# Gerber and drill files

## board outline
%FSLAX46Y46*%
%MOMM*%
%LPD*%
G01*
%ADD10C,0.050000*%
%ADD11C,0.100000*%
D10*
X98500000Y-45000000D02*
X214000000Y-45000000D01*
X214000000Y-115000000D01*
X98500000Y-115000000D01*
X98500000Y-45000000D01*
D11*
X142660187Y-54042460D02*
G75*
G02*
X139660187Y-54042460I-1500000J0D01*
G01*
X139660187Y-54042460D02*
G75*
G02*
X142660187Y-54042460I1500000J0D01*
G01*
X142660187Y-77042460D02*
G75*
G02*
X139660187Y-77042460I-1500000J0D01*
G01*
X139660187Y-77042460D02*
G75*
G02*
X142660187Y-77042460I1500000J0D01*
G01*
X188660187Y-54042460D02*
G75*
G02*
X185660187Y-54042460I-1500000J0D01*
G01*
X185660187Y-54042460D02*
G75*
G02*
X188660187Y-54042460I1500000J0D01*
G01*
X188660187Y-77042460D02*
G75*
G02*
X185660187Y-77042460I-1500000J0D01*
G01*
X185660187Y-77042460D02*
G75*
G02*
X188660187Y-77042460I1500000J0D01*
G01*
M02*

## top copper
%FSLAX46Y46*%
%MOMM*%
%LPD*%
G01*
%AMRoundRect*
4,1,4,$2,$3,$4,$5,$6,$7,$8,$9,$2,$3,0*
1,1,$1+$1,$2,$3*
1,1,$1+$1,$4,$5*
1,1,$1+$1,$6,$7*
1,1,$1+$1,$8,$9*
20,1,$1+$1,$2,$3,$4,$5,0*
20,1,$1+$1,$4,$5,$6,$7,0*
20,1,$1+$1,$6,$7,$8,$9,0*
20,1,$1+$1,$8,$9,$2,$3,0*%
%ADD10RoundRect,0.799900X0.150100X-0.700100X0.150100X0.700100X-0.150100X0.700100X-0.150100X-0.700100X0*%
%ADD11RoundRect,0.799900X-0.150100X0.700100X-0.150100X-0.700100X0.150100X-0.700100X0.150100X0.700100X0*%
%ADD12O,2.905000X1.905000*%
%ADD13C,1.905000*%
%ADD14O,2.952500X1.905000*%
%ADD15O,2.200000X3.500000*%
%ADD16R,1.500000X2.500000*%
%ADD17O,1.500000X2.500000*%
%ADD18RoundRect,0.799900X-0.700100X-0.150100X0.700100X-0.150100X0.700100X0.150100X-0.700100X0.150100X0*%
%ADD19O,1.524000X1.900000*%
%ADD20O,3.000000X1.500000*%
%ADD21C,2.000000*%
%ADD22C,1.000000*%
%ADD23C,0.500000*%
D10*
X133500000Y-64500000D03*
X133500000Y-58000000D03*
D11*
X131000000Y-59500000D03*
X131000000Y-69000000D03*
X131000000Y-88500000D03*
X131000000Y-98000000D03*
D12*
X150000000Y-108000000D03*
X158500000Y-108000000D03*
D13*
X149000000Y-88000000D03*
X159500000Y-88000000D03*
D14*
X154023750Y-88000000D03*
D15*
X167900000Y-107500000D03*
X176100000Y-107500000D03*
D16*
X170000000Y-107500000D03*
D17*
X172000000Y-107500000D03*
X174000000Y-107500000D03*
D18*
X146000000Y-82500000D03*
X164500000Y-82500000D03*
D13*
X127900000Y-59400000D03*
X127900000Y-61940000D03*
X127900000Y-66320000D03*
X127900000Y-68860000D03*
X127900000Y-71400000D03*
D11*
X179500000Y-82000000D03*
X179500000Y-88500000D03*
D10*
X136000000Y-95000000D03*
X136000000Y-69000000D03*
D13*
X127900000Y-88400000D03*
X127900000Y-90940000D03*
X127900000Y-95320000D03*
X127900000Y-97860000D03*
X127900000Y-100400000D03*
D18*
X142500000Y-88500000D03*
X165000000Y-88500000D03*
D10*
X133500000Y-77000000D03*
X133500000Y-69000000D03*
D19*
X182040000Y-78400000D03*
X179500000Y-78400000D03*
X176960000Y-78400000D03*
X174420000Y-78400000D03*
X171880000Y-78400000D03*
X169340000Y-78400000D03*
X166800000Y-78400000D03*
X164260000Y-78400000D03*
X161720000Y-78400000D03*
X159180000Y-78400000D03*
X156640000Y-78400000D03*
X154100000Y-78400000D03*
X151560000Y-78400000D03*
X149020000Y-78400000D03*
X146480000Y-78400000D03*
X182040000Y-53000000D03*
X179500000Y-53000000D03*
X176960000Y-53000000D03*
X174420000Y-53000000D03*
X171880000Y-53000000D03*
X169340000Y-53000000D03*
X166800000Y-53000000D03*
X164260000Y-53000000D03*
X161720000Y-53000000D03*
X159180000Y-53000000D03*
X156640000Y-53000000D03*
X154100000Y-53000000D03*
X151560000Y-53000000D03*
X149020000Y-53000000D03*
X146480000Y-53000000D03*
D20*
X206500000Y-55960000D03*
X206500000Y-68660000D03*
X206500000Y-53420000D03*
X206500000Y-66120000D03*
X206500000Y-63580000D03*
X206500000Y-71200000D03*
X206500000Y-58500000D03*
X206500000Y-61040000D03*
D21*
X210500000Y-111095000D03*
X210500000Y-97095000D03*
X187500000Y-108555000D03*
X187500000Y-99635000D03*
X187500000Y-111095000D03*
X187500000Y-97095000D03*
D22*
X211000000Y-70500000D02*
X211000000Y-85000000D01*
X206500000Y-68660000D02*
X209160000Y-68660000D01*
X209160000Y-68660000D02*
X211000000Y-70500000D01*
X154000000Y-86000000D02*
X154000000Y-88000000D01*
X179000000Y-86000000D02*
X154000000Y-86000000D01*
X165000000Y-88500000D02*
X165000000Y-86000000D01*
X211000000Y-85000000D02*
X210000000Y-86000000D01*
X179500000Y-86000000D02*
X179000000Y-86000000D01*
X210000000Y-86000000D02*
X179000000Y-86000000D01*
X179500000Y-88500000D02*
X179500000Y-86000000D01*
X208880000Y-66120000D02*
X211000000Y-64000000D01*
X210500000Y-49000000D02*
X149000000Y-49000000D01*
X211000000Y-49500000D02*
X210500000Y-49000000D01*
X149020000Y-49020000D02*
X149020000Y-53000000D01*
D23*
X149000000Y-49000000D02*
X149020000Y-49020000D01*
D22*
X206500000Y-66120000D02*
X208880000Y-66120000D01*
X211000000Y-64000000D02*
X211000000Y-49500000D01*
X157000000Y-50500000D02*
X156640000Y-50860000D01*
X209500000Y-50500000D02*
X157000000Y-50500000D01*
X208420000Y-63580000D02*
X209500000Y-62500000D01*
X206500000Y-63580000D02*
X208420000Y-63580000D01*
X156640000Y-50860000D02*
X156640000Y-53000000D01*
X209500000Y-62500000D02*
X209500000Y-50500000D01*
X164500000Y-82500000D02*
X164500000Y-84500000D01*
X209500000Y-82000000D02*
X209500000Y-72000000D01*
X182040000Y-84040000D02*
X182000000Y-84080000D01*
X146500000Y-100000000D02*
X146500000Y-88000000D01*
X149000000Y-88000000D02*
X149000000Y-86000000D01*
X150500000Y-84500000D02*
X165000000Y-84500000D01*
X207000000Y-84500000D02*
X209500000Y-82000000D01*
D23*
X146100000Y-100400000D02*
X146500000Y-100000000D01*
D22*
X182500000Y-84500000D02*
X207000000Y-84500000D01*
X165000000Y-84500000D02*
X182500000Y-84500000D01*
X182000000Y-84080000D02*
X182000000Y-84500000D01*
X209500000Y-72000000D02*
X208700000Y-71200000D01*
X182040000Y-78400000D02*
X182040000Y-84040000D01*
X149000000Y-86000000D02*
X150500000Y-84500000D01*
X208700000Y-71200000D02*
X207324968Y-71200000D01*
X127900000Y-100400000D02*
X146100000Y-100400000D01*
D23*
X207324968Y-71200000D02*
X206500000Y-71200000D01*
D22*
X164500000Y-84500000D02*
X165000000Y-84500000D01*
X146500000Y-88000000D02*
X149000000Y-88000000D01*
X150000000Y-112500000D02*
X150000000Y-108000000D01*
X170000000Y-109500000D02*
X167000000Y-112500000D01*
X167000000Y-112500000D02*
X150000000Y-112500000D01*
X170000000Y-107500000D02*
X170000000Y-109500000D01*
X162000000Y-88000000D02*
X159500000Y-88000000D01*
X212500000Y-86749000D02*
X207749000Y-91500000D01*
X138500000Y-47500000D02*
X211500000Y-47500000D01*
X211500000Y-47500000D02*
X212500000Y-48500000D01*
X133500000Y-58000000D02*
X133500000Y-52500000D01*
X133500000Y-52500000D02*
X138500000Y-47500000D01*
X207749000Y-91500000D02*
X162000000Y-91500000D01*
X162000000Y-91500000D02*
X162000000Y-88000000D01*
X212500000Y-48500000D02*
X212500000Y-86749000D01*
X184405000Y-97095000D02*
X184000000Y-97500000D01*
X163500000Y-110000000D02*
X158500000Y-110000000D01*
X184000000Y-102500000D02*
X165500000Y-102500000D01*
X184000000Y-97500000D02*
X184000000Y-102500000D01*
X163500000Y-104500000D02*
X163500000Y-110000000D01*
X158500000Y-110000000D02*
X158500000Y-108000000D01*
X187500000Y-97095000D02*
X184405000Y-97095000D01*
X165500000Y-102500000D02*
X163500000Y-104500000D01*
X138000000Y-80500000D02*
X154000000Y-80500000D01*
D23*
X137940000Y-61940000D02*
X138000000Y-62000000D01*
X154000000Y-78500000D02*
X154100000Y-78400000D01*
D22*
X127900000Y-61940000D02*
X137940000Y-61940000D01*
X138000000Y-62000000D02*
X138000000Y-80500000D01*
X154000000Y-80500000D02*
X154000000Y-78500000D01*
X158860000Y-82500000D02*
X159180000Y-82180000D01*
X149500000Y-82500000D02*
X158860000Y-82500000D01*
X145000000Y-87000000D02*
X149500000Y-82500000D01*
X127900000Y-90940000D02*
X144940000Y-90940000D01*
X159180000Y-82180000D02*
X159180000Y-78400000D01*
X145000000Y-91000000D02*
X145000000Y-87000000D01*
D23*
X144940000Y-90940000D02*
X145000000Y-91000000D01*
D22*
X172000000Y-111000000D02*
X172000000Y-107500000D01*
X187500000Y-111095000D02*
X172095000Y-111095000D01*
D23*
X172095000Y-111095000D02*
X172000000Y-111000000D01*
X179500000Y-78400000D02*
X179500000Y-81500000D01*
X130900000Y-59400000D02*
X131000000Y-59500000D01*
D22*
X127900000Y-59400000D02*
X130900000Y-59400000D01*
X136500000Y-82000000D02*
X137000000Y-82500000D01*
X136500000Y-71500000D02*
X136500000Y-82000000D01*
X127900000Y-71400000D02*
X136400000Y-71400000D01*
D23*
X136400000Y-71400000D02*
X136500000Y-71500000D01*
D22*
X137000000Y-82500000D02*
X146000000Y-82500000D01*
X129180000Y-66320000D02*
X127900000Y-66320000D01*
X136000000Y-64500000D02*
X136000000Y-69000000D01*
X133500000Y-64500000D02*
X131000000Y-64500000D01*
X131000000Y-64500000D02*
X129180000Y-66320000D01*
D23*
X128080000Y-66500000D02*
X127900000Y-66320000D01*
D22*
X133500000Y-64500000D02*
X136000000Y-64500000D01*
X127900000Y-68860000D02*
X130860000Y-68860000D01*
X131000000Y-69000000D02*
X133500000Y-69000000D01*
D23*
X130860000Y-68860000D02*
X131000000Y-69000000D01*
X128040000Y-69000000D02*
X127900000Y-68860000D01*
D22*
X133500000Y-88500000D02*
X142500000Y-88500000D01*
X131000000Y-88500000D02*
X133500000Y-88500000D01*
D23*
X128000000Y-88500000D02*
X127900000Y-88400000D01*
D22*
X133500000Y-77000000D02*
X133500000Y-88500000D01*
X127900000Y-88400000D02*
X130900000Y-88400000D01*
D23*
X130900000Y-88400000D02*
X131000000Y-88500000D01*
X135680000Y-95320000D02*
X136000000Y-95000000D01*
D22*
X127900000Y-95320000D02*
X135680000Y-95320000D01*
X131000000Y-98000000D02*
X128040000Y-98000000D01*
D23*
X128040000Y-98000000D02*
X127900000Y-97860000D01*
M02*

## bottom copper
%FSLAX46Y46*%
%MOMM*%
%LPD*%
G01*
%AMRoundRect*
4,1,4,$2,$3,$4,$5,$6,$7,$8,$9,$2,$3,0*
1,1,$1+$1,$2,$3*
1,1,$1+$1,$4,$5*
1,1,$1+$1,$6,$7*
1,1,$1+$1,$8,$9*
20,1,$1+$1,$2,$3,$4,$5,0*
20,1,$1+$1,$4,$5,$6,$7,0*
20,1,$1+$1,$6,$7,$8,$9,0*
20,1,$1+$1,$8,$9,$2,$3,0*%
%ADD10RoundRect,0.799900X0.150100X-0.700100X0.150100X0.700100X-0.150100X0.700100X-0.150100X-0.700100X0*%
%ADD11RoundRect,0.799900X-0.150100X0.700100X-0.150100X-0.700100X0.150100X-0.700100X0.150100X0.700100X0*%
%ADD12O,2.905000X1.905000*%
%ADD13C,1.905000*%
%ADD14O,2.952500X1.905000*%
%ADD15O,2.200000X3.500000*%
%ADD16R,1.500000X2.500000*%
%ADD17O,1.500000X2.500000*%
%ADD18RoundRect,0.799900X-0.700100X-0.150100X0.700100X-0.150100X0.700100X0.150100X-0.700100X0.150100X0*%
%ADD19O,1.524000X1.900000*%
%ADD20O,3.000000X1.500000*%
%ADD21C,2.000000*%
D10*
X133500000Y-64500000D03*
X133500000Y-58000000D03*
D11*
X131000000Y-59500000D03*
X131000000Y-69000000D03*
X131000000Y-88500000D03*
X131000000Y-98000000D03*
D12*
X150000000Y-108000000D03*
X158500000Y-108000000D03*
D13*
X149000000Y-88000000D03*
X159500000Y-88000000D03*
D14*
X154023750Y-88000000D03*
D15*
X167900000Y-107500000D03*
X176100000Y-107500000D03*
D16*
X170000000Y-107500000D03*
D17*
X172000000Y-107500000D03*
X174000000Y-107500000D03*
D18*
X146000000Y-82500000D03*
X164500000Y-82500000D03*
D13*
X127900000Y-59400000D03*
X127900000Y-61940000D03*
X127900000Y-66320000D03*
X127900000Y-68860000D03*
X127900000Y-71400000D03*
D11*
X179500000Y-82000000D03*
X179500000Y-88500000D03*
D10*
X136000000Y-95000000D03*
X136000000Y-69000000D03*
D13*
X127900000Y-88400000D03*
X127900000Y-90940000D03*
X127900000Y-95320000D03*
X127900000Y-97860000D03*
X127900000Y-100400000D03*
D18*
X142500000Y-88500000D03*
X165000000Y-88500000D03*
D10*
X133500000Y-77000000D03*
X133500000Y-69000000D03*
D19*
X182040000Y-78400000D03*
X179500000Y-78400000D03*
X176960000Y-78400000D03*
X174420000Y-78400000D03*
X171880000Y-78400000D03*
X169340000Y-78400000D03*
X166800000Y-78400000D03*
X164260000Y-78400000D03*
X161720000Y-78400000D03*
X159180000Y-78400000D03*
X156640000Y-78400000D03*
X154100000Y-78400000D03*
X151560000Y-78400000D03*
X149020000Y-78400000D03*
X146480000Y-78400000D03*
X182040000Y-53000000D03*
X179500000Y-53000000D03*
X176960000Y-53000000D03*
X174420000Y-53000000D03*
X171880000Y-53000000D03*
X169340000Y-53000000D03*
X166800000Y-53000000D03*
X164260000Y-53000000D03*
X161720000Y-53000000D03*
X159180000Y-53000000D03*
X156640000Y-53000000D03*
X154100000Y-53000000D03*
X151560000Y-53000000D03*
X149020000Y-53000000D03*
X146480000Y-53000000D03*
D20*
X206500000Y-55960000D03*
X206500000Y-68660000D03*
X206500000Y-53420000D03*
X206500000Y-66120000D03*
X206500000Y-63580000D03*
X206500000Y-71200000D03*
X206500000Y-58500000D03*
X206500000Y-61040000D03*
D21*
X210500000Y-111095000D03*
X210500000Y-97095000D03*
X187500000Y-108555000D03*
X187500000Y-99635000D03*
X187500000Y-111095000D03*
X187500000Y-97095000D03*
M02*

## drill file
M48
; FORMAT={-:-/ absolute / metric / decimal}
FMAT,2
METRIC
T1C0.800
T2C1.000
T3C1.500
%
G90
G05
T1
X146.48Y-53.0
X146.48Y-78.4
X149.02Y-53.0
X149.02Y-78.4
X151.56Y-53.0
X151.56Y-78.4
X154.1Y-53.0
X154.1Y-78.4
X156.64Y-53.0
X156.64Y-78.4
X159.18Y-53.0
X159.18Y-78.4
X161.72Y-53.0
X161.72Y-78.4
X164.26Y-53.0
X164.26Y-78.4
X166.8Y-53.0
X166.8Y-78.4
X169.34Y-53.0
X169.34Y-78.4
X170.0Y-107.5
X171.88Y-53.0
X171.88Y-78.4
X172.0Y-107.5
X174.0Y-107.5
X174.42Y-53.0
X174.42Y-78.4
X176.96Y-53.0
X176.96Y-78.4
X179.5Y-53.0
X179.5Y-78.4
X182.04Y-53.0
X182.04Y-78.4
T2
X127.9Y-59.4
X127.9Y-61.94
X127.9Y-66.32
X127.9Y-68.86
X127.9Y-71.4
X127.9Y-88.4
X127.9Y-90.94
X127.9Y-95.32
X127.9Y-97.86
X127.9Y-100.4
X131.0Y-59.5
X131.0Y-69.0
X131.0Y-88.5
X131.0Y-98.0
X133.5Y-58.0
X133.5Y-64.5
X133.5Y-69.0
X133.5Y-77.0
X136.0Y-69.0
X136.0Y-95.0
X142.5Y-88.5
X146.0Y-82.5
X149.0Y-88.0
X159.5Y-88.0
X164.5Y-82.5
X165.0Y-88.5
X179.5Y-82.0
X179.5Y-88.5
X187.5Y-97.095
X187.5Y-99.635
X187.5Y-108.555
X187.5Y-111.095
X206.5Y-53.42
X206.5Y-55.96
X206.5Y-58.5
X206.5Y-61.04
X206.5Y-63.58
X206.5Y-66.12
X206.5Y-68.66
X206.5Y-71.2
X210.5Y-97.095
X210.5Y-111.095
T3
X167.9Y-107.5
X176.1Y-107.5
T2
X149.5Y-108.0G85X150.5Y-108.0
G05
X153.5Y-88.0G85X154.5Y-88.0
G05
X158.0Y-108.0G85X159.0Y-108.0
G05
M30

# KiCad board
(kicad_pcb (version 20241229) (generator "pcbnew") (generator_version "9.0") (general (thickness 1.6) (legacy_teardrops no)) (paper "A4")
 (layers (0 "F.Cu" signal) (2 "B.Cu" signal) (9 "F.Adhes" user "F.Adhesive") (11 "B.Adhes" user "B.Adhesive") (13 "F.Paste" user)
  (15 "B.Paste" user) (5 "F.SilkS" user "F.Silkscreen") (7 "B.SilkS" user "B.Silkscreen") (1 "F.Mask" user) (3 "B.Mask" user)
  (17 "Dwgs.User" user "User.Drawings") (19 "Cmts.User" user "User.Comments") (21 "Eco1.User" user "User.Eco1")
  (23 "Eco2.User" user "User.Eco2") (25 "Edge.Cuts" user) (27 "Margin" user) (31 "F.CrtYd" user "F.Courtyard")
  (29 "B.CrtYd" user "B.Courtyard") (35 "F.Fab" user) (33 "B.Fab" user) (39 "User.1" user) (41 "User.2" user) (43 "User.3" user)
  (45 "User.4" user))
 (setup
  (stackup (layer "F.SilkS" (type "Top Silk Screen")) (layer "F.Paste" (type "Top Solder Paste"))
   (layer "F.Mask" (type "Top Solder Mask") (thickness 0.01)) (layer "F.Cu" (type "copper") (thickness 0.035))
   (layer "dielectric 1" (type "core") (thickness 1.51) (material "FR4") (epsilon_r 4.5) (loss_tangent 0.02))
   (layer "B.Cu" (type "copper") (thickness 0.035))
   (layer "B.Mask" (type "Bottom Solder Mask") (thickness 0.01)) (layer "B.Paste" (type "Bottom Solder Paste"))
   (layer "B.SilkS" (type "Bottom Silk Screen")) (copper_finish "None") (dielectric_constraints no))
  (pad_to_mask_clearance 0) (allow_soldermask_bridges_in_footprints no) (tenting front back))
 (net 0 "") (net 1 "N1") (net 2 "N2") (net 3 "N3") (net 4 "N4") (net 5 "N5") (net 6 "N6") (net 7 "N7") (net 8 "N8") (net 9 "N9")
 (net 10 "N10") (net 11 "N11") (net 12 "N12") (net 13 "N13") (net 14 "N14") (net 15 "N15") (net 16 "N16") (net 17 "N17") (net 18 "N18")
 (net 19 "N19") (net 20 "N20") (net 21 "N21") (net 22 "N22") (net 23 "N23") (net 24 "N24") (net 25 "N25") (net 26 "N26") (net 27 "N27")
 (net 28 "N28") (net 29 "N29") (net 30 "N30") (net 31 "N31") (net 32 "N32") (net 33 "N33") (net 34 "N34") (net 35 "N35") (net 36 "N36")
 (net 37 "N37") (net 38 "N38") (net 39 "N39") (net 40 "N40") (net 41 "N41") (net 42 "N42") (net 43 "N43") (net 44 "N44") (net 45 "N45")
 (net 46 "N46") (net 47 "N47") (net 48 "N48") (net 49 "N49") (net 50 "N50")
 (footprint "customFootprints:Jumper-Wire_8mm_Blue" (layer "F.Cu") (at 133.5 66 90)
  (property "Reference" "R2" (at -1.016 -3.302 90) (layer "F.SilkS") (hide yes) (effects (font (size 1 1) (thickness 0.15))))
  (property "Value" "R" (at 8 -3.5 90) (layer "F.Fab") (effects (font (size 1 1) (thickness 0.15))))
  (pad "1" thru_hole roundrect (at 1.5 0 90) (size 3 1.9) (drill 1) (layers "*.Cu") (remove_unused_layers no) (roundrect_rratio 0.421)
   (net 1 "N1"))
  (pad "2" thru_hole roundrect (at 8 0 90) (size 3 1.9) (drill 1) (layers "*.Cu") (remove_unused_layers no) (roundrect_rratio 0.421)
   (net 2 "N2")))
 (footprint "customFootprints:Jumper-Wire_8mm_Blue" (layer "F.Cu") (at 131 59.5 -90)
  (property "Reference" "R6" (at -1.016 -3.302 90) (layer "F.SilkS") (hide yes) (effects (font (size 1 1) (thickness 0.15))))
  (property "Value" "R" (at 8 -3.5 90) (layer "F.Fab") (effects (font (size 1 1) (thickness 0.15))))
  (pad "1" thru_hole roundrect (at 0 0 270) (size 3 1.9) (drill 1) (layers "*.Cu") (remove_unused_layers no) (roundrect_rratio 0.421)
   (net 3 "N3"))
  (pad "2" thru_hole roundrect (at 9.5 0 270) (size 3 1.9) (drill 1) (layers "*.Cu") (remove_unused_layers no) (roundrect_rratio 0.421)
   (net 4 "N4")))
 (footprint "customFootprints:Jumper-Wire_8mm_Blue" (layer "F.Cu") (at 131 88.5 -90)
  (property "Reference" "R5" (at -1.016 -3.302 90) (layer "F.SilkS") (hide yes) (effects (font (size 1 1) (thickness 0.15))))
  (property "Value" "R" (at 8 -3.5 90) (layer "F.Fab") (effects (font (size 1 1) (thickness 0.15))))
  (pad "1" thru_hole roundrect (at 0 0 270) (size 3 1.9) (drill 1) (layers "*.Cu") (remove_unused_layers no) (roundrect_rratio 0.421)
   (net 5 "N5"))
  (pad "2" thru_hole roundrect (at 9.5 0 270) (size 3 1.9) (drill 1) (layers "*.Cu") (remove_unused_layers no) (roundrect_rratio 0.421)
   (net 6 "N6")))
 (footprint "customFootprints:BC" (layer "F.Cu") (at 154.5 98 90)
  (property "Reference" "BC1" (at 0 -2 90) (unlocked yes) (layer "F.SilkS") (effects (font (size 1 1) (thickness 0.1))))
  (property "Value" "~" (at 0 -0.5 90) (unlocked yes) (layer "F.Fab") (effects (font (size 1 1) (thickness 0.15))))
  (pad "1" thru_hole oval (at -10 -4.5 90) (size 1.905 2.905) (drill oval 1 2) (layers "*.Cu" "*.Mask") (remove_unused_layers no)
   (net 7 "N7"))
  (pad "2" thru_hole oval (at -10 4 90) (size 1.905 2.905) (drill oval 1 2) (layers "*.Cu" "*.Mask") (remove_unused_layers no) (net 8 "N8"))
  (pad "3" thru_hole circle (at 10 -5.5 90) (size 1.905 1.905) (drill 1) (layers "*.Cu" "*.Mask") (remove_unused_layers no) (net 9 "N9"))
  (pad "4" thru_hole circle (at 10 5 90) (size 1.905 1.905) (drill 1) (layers "*.Cu" "*.Mask") (remove_unused_layers no) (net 2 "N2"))
  (pad "5" thru_hole oval (at 10 -0.5 90) (size 1.905 2.9525) (drill oval 1 2 (offset 0 0.02375)) (layers "*.Cu" "*.Mask")
   (remove_unused_layers no) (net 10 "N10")))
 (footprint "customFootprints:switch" (layer "F.Cu") (at 170 107.5)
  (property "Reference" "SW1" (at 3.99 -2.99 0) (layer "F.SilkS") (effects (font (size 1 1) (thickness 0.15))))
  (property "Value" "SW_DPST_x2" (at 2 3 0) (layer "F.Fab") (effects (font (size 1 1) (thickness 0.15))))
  (pad "" thru_hole oval (at -2.1 0) (size 2.2 3.5) (drill 1.5) (layers "*.Cu" "*.Mask") (remove_unused_layers no))
  (pad "" thru_hole oval (at 6.1 0) (size 2.2 3.5) (drill 1.5) (layers "*.Cu" "*.Mask") (remove_unused_layers no))
  (pad "1" thru_hole rect (at 0 0) (size 1.5 2.5) (drill 0.8) (layers "*.Cu" "*.Mask") (remove_unused_layers no) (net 7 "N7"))
  (pad "2" thru_hole oval (at 2 0) (size 1.5 2.5) (drill 0.8) (layers "*.Cu" "*.Mask") (remove_unused_layers no) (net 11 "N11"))
  (pad "3" thru_hole oval (at 4 0) (size 1.5 2.5) (drill 0.8) (layers "*.Cu" "*.Mask") (remove_unused_layers no)))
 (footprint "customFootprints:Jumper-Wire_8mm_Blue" (layer "F.Cu") (at 146 82.5)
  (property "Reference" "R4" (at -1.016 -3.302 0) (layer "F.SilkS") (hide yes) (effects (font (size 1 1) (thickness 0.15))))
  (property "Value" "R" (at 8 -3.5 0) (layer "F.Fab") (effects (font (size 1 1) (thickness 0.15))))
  (pad "1" thru_hole roundrect (at 0 0) (size 3 1.9) (drill 1) (layers "*.Cu") (remove_unused_layers no) (roundrect_rratio 0.421)
   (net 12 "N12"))
  (pad "2" thru_hole roundrect (at 18.5 0) (size 3 1.9) (drill 1) (layers "*.Cu") (remove_unused_layers no) (roundrect_rratio 0.421)
   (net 9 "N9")))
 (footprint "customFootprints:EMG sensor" (layer "F.Cu") (at 129.4 79.4 180)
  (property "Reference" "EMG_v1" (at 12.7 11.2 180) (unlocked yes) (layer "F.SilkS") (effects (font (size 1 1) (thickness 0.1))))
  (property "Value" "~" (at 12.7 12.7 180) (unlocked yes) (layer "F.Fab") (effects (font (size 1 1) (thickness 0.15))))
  (pad "1" thru_hole circle (at 1.5 20 180) (size 1.905 1.905) (drill 1) (layers "*.Cu" "*.Mask") (remove_unused_layers no) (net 3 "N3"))
  (pad "2" thru_hole circle (at 1.5 17.46 180) (size 1.905 1.905) (drill 1) (layers "*.Cu" "*.Mask") (remove_unused_layers no)
   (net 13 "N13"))
  (pad "3" thru_hole circle (at 1.5 13.08 180) (size 1.905 1.905) (drill 1) (layers "*.Cu" "*.Mask") (remove_unused_layers no) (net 1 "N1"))
  (pad "4" thru_hole circle (at 1.5 10.54 180) (size 1.905 1.905) (drill 1) (layers "*.Cu" "*.Mask") (remove_unused_layers no) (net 4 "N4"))
  (pad "5" thru_hole circle (at 1.5 8 180) (size 1.905 1.905) (drill 1) (layers "*.Cu" "*.Mask") (remove_unused_layers no) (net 12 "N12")))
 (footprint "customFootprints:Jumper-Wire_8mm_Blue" (layer "F.Cu") (at 179.5 80.5 -90)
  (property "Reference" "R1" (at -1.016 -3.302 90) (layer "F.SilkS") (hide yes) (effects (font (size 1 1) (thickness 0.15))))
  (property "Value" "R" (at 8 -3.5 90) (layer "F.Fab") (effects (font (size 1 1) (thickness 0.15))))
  (pad "1" thru_hole roundrect (at 1.5 0 270) (size 3 1.9) (drill 1) (layers "*.Cu") (remove_unused_layers no) (roundrect_rratio 0.421)
   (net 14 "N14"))
  (pad "2" thru_hole roundrect (at 8 0 270) (size 3 1.9) (drill 1) (layers "*.Cu") (remove_unused_layers no) (roundrect_rratio 0.421)
   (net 10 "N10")))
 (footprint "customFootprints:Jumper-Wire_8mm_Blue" (layer "F.Cu") (at 136 95 90)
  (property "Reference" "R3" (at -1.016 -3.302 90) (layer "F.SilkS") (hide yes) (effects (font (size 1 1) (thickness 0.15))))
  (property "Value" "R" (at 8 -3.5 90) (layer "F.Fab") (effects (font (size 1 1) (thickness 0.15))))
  (pad "1" thru_hole roundrect (at 0 0 90) (size 3 1.9) (drill 1) (layers "*.Cu") (remove_unused_layers no) (roundrect_rratio 0.421)
   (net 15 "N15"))
  (pad "2" thru_hole roundrect (at 26 0 90) (size 3 1.9) (drill 1) (layers "*.Cu") (remove_unused_layers no) (roundrect_rratio 0.421)
   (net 1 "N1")))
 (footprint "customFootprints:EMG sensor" (layer "F.Cu") (at 129.4 108.4 180)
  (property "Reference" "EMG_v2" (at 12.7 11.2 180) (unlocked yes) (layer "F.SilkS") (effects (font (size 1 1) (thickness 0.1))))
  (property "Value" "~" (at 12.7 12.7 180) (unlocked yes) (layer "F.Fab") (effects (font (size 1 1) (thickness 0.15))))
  (pad "1" thru_hole circle (at 1.5 20 180) (size 1.905 1.905) (drill 1) (layers "*.Cu" "*.Mask") (remove_unused_layers no) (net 5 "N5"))
  (pad "2" thru_hole circle (at 1.5 17.46 180) (size 1.905 1.905) (drill 1) (layers "*.Cu" "*.Mask") (remove_unused_layers no)
   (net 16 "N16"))
  (pad "3" thru_hole circle (at 1.5 13.08 180) (size 1.905 1.905) (drill 1) (layers "*.Cu" "*.Mask") (remove_unused_layers no)
   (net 15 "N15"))
  (pad "4" thru_hole circle (at 1.5 10.54 180) (size 1.905 1.905) (drill 1) (layers "*.Cu" "*.Mask") (remove_unused_layers no) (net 6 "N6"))
  (pad "5" thru_hole circle (at 1.5 8 180) (size 1.905 1.905) (drill 1) (layers "*.Cu" "*.Mask") (remove_unused_layers no) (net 9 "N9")))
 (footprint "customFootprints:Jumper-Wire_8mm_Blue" (layer "F.Cu") (at 142.5 88.5)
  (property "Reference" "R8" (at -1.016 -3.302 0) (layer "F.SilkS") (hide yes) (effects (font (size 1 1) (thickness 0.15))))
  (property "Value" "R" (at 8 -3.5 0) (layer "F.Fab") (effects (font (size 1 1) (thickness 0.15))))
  (pad "1" thru_hole roundrect (at 0 0) (size 3 1.9) (drill 1) (layers "*.Cu") (remove_unused_layers no) (roundrect_rratio 0.421)
   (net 5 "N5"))
  (pad "2" thru_hole roundrect (at 22.5 0) (size 3 1.9) (drill 1) (layers "*.Cu") (remove_unused_layers no) (roundrect_rratio 0.421)
   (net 10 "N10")))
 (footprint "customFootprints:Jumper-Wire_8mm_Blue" (layer "F.Cu") (at 133.5 77 90)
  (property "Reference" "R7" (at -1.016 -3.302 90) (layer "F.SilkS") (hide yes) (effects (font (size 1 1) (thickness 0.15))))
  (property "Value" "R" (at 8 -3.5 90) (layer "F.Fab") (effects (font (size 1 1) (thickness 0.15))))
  (pad "1" thru_hole roundrect (at 0 0 90) (size 3 1.9) (drill 1) (layers "*.Cu") (remove_unused_layers no) (roundrect_rratio 0.421)
   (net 5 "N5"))
  (pad "2" thru_hole roundrect (at 8 0 90) (size 3 1.9) (drill 1) (layers "*.Cu") (remove_unused_layers no) (roundrect_rratio 0.421)
   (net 4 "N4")))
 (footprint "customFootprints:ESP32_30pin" (layer "F.Cu") (at 164.020187 65.47246)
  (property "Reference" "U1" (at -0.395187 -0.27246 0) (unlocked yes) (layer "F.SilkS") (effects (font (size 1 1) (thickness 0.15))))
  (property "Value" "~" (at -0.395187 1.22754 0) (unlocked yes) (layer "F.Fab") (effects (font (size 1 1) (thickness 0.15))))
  (fp_circle (center -22.86 -11.43) (end -21.36 -11.43) (stroke (width 0.1) (type default)) (fill no) (layer "Edge.Cuts"))
  (fp_circle (center -22.86 11.57) (end -21.36 11.57) (stroke (width 0.1) (type default)) (fill no) (layer "Edge.Cuts"))
  (fp_circle (center 23.14 -11.43) (end 24.64 -11.43) (stroke (width 0.1) (type default)) (fill no) (layer "Edge.Cuts"))
  (fp_circle (center 23.14 11.57) (end 24.64 11.57) (stroke (width 0.1) (type default)) (fill no) (layer "Edge.Cuts"))
  (pad "1" thru_hole oval (at 18.019813 12.92754) (size 1.524 1.9) (drill 0.8) (layers "*.Cu" "*.Mask") (remove_unused_layers no)
   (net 9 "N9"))
  (pad "2" thru_hole oval (at 15.479813 12.92754) (size 1.524 1.9) (drill 0.8) (layers "*.Cu" "*.Mask") (remove_unused_layers no)
   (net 14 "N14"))
  (pad "3" thru_hole oval (at 12.939813 12.92754) (size 1.524 1.9) (drill 0.8) (layers "*.Cu" "*.Mask") (remove_unused_layers no)
   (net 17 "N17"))
  (pad "4" thru_hole oval (at 10.399813 12.92754) (size 1.524 1.9) (drill 0.8) (layers "*.Cu" "*.Mask") (remove_unused_layers no)
   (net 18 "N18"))
  (pad "5" thru_hole oval (at 7.859813 12.92754) (size 1.524 1.9) (drill 0.8) (layers "*.Cu" "*.Mask") (remove_unused_layers no)
   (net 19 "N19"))
  (pad "6" thru_hole oval (at 5.319813 12.92754) (size 1.524 1.9) (drill 0.8) (layers "*.Cu" "*.Mask") (remove_unused_layers no)
   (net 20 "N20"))
  (pad "7" thru_hole oval (at 2.779813 12.92754) (size 1.524 1.9) (drill 0.8) (layers "*.Cu" "*.Mask") (remove_unused_layers no)
   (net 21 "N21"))
  (pad "8" thru_hole oval (at 0.239813 12.92754) (size 1.524 1.9) (drill 0.8) (layers "*.Cu" "*.Mask") (remove_unused_layers no)
   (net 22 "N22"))
  (pad "9" thru_hole oval (at -2.300187 12.92754) (size 1.524 1.9) (drill 0.8) (layers "*.Cu" "*.Mask") (remove_unused_layers no)
   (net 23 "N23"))
  (pad "10" thru_hole oval (at -4.840187 12.92754) (size 1.524 1.9) (drill 0.8) (layers "*.Cu" "*.Mask") (remove_unused_layers no)
   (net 16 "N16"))
  (pad "11" thru_hole oval (at -7.380187 12.92754) (size 1.524 1.9) (drill 0.8) (layers "*.Cu" "*.Mask") (remove_unused_layers no)
   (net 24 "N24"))
  (pad "12" thru_hole oval (at -9.920187 12.92754) (size 1.524 1.9) (drill 0.8) (layers "*.Cu" "*.Mask") (remove_unused_layers no)
   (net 13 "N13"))
  (pad "13" thru_hole oval (at -12.460187 12.92754) (size 1.524 1.9) (drill 0.8) (layers "*.Cu" "*.Mask") (remove_unused_layers no)
   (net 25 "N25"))
  (pad "14" thru_hole oval (at -15.000187 12.92754) (size 1.524 1.9) (drill 0.8) (layers "*.Cu" "*.Mask") (remove_unused_layers no)
   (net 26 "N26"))
  (pad "15" thru_hole oval (at -17.540187 12.92754) (size 1.524 1.9) (drill 0.8) (layers "*.Cu" "*.Mask") (remove_unused_layers no)
   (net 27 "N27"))
  (pad "16" thru_hole oval (at 18.019813 -12.47246) (size 1.524 1.9) (drill 0.8) (layers "*.Cu" "*.Mask") (remove_unused_layers no)
   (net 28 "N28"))
  (pad "17" thru_hole oval (at 15.479813 -12.47246) (size 1.524 1.9) (drill 0.8) (layers "*.Cu" "*.Mask") (remove_unused_layers no)
   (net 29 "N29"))
  (pad "18" thru_hole oval (at 12.939813 -12.47246) (size 1.524 1.9) (drill 0.8) (layers "*.Cu" "*.Mask") (remove_unused_layers no)
   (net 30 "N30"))
  (pad "19" thru_hole oval (at 10.399813 -12.47246) (size 1.524 1.9) (drill 0.8) (layers "*.Cu" "*.Mask") (remove_unused_layers no)
   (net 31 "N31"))
  (pad "20" thru_hole oval (at 7.859813 -12.47246) (size 1.524 1.9) (drill 0.8) (layers "*.Cu" "*.Mask") (remove_unused_layers no)
   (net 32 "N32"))
  (pad "21" thru_hole oval (at 5.319813 -12.47246) (size 1.524 1.9) (drill 0.8) (layers "*.Cu" "*.Mask") (remove_unused_layers no)
   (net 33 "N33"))
  (pad "22" thru_hole oval (at 2.779813 -12.47246) (size 1.524 1.9) (drill 0.8) (layers "*.Cu" "*.Mask") (remove_unused_layers no)
   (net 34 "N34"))
  (pad "23" thru_hole oval (at 0.239813 -12.47246) (size 1.524 1.9) (drill 0.8) (layers "*.Cu" "*.Mask") (remove_unused_layers no)
   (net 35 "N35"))
  (pad "24" thru_hole oval (at -2.300187 -12.47246) (size 1.524 1.9) (drill 0.8) (layers "*.Cu" "*.Mask") (remove_unused_layers no)
   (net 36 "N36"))
  (pad "25" thru_hole oval (at -4.840187 -12.47246) (size 1.524 1.9) (drill 0.8) (layers "*.Cu" "*.Mask") (remove_unused_layers no)
   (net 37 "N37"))
  (pad "26" thru_hole oval (at -7.380187 -12.47246) (size 1.524 1.9) (drill 0.8) (layers "*.Cu" "*.Mask") (remove_unused_layers no)
   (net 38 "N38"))
  (pad "27" thru_hole oval (at -9.920187 -12.47246) (size 1.524 1.9) (drill 0.8) (layers "*.Cu" "*.Mask") (remove_unused_layers no)
   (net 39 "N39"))
  (pad "28" thru_hole oval (at -12.460187 -12.47246) (size 1.524 1.9) (drill 0.8) (layers "*.Cu" "*.Mask") (remove_unused_layers no)
   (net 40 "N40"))
  (pad "29" thru_hole oval (at -15.000187 -12.47246) (size 1.524 1.9) (drill 0.8) (layers "*.Cu" "*.Mask") (remove_unused_layers no)
   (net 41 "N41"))
  (pad "30" thru_hole oval (at -17.540187 -12.47246) (size 1.524 1.9) (drill 0.8) (layers "*.Cu" "*.Mask") (remove_unused_layers no)
   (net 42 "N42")))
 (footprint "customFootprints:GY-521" (layer "F.Cu") (at 208.27 51.356 180)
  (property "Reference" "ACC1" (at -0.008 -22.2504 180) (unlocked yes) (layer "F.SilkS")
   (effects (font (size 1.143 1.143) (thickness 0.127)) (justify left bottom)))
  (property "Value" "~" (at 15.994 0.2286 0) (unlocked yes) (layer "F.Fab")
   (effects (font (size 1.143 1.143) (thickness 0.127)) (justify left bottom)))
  (pad "AD0" thru_hole oval (at 1.77 -4.604 180) (size 3 1.5) (drill 1) (layers "*.Cu" "*.Mask") (remove_unused_layers no) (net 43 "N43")
   (solder_mask_margin 0.1016) (thermal_bridge_angle 0))
  (pad "GND" thru_hole oval (at 1.77 -17.304 180) (size 3 1.5) (drill 1) (layers "*.Cu" "*.Mask") (remove_unused_layers no) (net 10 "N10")
   (solder_mask_margin 0.1016) (thermal_bridge_angle 0))
  (pad "INT" thru_hole oval (at 1.77 -2.064 180) (size 3 1.5) (drill 1) (layers "*.Cu" "*.Mask") (remove_unused_layers no) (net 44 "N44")
   (solder_mask_margin 0.1016) (thermal_bridge_angle 0))
  (pad "SCL" thru_hole oval (at 1.77 -14.764 180) (size 3 1.5) (drill 1) (layers "*.Cu" "*.Mask") (remove_unused_layers no) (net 41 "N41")
   (solder_mask_margin 0.1016) (thermal_bridge_angle 0))
  (pad "SDA" thru_hole oval (at 1.77 -12.224 180) (size 3 1.5) (drill 1) (layers "*.Cu" "*.Mask") (remove_unused_layers no) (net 38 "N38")
   (solder_mask_margin 0.1016) (thermal_bridge_angle 0))
  (pad "VCC" thru_hole oval (at 1.77 -19.844 180) (size 3 1.5) (drill 1) (layers "*.Cu" "*.Mask") (remove_unused_layers no) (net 9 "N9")
   (solder_mask_margin 0.1016) (thermal_bridge_angle 0))
  (pad "XCL" thru_hole oval (at 1.77 -7.144 180) (size 3 1.5) (drill 1) (layers "*.Cu" "*.Mask") (remove_unused_layers no) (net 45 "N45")
   (solder_mask_margin 0.1016) (thermal_bridge_angle 0))
  (pad "XDA" thru_hole oval (at 1.77 -9.684 180) (size 3 1.5) (drill 1) (layers "*.Cu" "*.Mask") (remove_unused_layers no) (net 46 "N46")
   (solder_mask_margin 0.1016) (thermal_bridge_angle 0)))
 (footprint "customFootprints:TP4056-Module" (layer "F.Cu") (at 213 95.495 180)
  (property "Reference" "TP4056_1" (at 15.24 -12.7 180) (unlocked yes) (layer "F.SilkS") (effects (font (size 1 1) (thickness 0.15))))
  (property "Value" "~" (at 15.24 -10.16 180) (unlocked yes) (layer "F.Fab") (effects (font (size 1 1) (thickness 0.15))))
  (pad "1" thru_hole circle (at 2.5 -15.6 180) (size 2 2) (drill 1) (layers "*.Cu" "*.Mask") (remove_unused_layers no) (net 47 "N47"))
  (pad "2" thru_hole circle (at 2.5 -1.6 180) (size 2 2) (drill 1) (layers "*.Cu" "*.Mask") (remove_unused_layers no) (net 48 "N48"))
  (pad "3" thru_hole circle (at 25.5 -13.06 180) (size 2 2) (drill 1) (layers "*.Cu" "*.Mask") (remove_unused_layers no) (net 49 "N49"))
  (pad "4" thru_hole circle (at 25.5 -4.14 180) (size 2 2) (drill 1) (layers "*.Cu" "*.Mask") (remove_unused_layers no) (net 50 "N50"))
  (pad "5" thru_hole circle (at 25.5 -15.6 180) (size 2 2) (drill 1) (layers "*.Cu" "*.Mask") (remove_unused_layers no) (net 11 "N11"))
  (pad "6" thru_hole circle (at 25.5 -1.6 180) (size 2 2) (drill 1) (layers "*.Cu" "*.Mask") (remove_unused_layers no) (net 8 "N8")))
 (gr_rect (start 98.5 45) (end 214 115) (stroke (width 0.05) (type default)) (fill no) (layer "Edge.Cuts"))
 (segment (start 211 70.5) (end 211 85) (width 1) (layer "F.Cu") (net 10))
 (segment (start 206.5 68.66) (end 209.16 68.66) (width 1) (layer "F.Cu") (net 10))
 (segment (start 209.16 68.66) (end 211 70.5) (width 1) (layer "F.Cu") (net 10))
 (segment (start 154 86) (end 154 88) (width 1) (layer "F.Cu") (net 10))
 (segment (start 179 86) (end 154 86) (width 1) (layer "F.Cu") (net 10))
 (segment (start 165 88.5) (end 165 86) (width 1) (layer "F.Cu") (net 10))
 (segment (start 211 85) (end 210 86) (width 1) (layer "F.Cu") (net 10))
 (segment (start 179.5 86) (end 179 86) (width 1) (layer "F.Cu") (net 10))
 (segment (start 210 86) (end 179 86) (width 1) (layer "F.Cu") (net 10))
 (segment (start 179.5 88.5) (end 179.5 86) (width 1) (layer "F.Cu") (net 10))
 (segment (start 208.88 66.12) (end 211 64) (width 1) (layer "F.Cu") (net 41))
 (segment (start 210.5 49) (end 149 49) (width 1) (layer "F.Cu") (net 41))
 (segment (start 211 49.5) (end 210.5 49) (width 1) (layer "F.Cu") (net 41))
 (segment (start 149.02 49.02) (end 149.02 53) (width 1) (layer "F.Cu") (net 41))
 (segment (start 149 49) (end 149.02 49.02) (width 0.5) (layer "F.Cu") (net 41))
 (segment (start 206.5 66.12) (end 208.88 66.12) (width 1) (layer "F.Cu") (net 41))
 (segment (start 211 64) (end 211 49.5) (width 1) (layer "F.Cu") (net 41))
 (segment (start 157 50.5) (end 156.64 50.86) (width 1) (layer "F.Cu") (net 38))
 (segment (start 209.5 50.5) (end 157 50.5) (width 1) (layer "F.Cu") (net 38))
 (segment (start 208.42 63.58) (end 209.5 62.5) (width 1) (layer "F.Cu") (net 38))
 (segment (start 206.5 63.58) (end 208.42 63.58) (width 1) (layer "F.Cu") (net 38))
 (segment (start 156.64 50.86) (end 156.64 53) (width 1) (layer "F.Cu") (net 38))
 (segment (start 209.5 62.5) (end 209.5 50.5) (width 1) (layer "F.Cu") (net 38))
 (segment (start 164.5 82.5) (end 164.5 84.5) (width 1) (layer "F.Cu") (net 9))
 (segment (start 209.5 82) (end 209.5 72) (width 1) (layer "F.Cu") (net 9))
 (segment (start 182.04 84.04) (end 182 84.08) (width 1) (layer "F.Cu") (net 9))
 (segment (start 146.5 100) (end 146.5 88) (width 1) (layer "F.Cu") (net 9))
 (segment (start 149 88) (end 149 86) (width 1) (layer "F.Cu") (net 9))
 (segment (start 150.5 84.5) (end 165 84.5) (width 1) (layer "F.Cu") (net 9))
 (segment (start 207 84.5) (end 209.5 82) (width 1) (layer "F.Cu") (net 9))
 (segment (start 146.1 100.4) (end 146.5 100) (width 0.5) (layer "F.Cu") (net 9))
 (segment (start 182.5 84.5) (end 207 84.5) (width 1) (layer "F.Cu") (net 9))
 (segment (start 165 84.5) (end 182.5 84.5) (width 1) (layer "F.Cu") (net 9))
 (segment (start 182 84.08) (end 182 84.5) (width 1) (layer "F.Cu") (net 9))
 (segment (start 209.5 72) (end 208.7 71.2) (width 1) (layer "F.Cu") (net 9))
 (segment (start 182.04 78.4) (end 182.04 84.04) (width 1) (layer "F.Cu") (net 9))
 (segment (start 149 86) (end 150.5 84.5) (width 1) (layer "F.Cu") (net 9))
 (segment (start 208.7 71.2) (end 207.324968 71.2) (width 1) (layer "F.Cu") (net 9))
 (segment (start 127.9 100.4) (end 146.1 100.4) (width 1) (layer "F.Cu") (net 9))
 (segment (start 207.324968 71.2) (end 206.5 71.2) (width 0.5) (layer "F.Cu") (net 9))
 (segment (start 164.5 84.5) (end 165 84.5) (width 1) (layer "F.Cu") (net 9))
 (segment (start 146.5 88) (end 149 88) (width 1) (layer "F.Cu") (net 9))
 (segment (start 150 112.5) (end 150 108) (width 1) (layer "F.Cu") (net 7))
 (segment (start 170 109.5) (end 167 112.5) (width 1) (layer "F.Cu") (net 7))
 (segment (start 167 112.5) (end 150 112.5) (width 1) (layer "F.Cu") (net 7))
 (segment (start 170 107.5) (end 170 109.5) (width 1) (layer "F.Cu") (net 7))
 (segment (start 162 88) (end 159.5 88) (width 1) (layer "F.Cu") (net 2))
 (segment (start 212.5 86.749) (end 207.749 91.5) (width 1) (layer "F.Cu") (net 2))
 (segment (start 138.5 47.5) (end 211.5 47.5) (width 1) (layer "F.Cu") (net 2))
 (segment (start 211.5 47.5) (end 212.5 48.5) (width 1) (layer "F.Cu") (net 2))
 (segment (start 133.5 58) (end 133.5 52.5) (width 1) (layer "F.Cu") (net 2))
 (segment (start 133.5 52.5) (end 138.5 47.5) (width 1) (layer "F.Cu") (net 2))
 (segment (start 207.749 91.5) (end 162 91.5) (width 1) (layer "F.Cu") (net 2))
 (segment (start 162 91.5) (end 162 88) (width 1) (layer "F.Cu") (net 2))
 (segment (start 212.5 48.5) (end 212.5 86.749) (width 1) (layer "F.Cu") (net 2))
 (segment (start 184.405 97.095) (end 184 97.5) (width 1) (layer "F.Cu") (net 8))
 (segment (start 163.5 110) (end 158.5 110) (width 1) (layer "F.Cu") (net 8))
 (segment (start 184 102.5) (end 165.5 102.5) (width 1) (layer "F.Cu") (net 8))
 (segment (start 184 97.5) (end 184 102.5) (width 1) (layer "F.Cu") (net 8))
 (segment (start 163.5 104.5) (end 163.5 110) (width 1) (layer "F.Cu") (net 8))
 (segment (start 158.5 110) (end 158.5 108) (width 1) (layer "F.Cu") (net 8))
 (segment (start 187.5 97.095) (end 184.405 97.095) (width 1) (layer "F.Cu") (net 8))
 (segment (start 165.5 102.5) (end 163.5 104.5) (width 1) (layer "F.Cu") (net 8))
 (segment (start 138 80.5) (end 154 80.5) (width 1) (layer "F.Cu") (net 13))
 (segment (start 137.94 61.94) (end 138 62) (width 0.5) (layer "F.Cu") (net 13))
 (segment (start 154 78.5) (end 154.1 78.4) (width 0.5) (layer "F.Cu") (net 13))
 (segment (start 127.9 61.94) (end 137.94 61.94) (width 1) (layer "F.Cu") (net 13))
 (segment (start 138 62) (end 138 80.5) (width 1) (layer "F.Cu") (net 13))
 (segment (start 154 80.5) (end 154 78.5) (width 1) (layer "F.Cu") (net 13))
 (segment (start 158.86 82.5) (end 159.18 82.18) (width 1) (layer "F.Cu") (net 16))
 (segment (start 149.5 82.5) (end 158.86 82.5) (width 1) (layer "F.Cu") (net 16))
 (segment (start 145 87) (end 149.5 82.5) (width 1) (layer "F.Cu") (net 16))
 (segment (start 127.9 90.94) (end 144.94 90.94) (width 1) (layer "F.Cu") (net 16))
 (segment (start 159.18 82.18) (end 159.18 78.4) (width 1) (layer "F.Cu") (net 16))
 (segment (start 145 91) (end 145 87) (width 1) (layer "F.Cu") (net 16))
 (segment (start 144.94 90.94) (end 145 91) (width 0.5) (layer "F.Cu") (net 16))
 (segment (start 172 111) (end 172 107.5) (width 1) (layer "F.Cu") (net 11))
 (segment (start 187.5 111.095) (end 172.095 111.095) (width 1) (layer "F.Cu") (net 11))
 (segment (start 172.095 111.095) (end 172 111) (width 0.5) (layer "F.Cu") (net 11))
 (segment (start 179.5 78.4) (end 179.5 81.5) (width 0.5) (layer "F.Cu") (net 14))
 (segment (start 130.9 59.4) (end 131 59.5) (width 0.5) (layer "F.Cu") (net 3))
 (segment (start 127.9 59.4) (end 130.9 59.4) (width 1) (layer "F.Cu") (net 3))
 (segment (start 136.5 82) (end 137 82.5) (width 1) (layer "F.Cu") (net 12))
 (segment (start 136.5 71.5) (end 136.5 82) (width 1) (layer "F.Cu") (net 12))
 (segment (start 127.9 71.4) (end 136.4 71.4) (width 1) (layer "F.Cu") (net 12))
 (segment (start 136.4 71.4) (end 136.5 71.5) (width 0.5) (layer "F.Cu") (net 12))
 (segment (start 137 82.5) (end 146 82.5) (width 1) (layer "F.Cu") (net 12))
 (segment (start 129.18 66.32) (end 127.9 66.32) (width 1) (layer "F.Cu") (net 1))
 (segment (start 136 64.5) (end 136 69) (width 1) (layer "F.Cu") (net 1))
 (segment (start 133.5 64.5) (end 131 64.5) (width 1) (layer "F.Cu") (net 1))
 (segment (start 131 64.5) (end 129.18 66.32) (width 1) (layer "F.Cu") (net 1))
 (segment (start 128.08 66.5) (end 127.9 66.32) (width 0.5) (layer "F.Cu") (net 1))
 (segment (start 133.5 64.5) (end 136 64.5) (width 1) (layer "F.Cu") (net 1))
 (segment (start 127.9 68.86) (end 130.86 68.86) (width 1) (layer "F.Cu") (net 4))
 (segment (start 131 69) (end 133.5 69) (width 1) (layer "F.Cu") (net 4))
 (segment (start 130.86 68.86) (end 131 69) (width 0.5) (layer "F.Cu") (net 4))
 (segment (start 128.04 69) (end 127.9 68.86) (width 0.5) (layer "F.Cu") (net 4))
 (segment (start 133.5 88.5) (end 142.5 88.5) (width 1) (layer "F.Cu") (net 5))
 (segment (start 131 88.5) (end 133.5 88.5) (width 1) (layer "F.Cu") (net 5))
 (segment (start 128 88.5) (end 127.9 88.4) (width 0.5) (layer "F.Cu") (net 5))
 (segment (start 133.5 77) (end 133.5 88.5) (width 1) (layer "F.Cu") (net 5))
 (segment (start 127.9 88.4) (end 130.9 88.4) (width 1) (layer "F.Cu") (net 5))
 (segment (start 130.9 88.4) (end 131 88.5) (width 0.5) (layer "F.Cu") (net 5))
 (segment (start 135.68 95.32) (end 136 95) (width 0.5) (layer "F.Cu") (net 15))
 (segment (start 127.9 95.32) (end 135.68 95.32) (width 1) (layer "F.Cu") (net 15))
 (segment (start 131 98) (end 128.04 98) (width 1) (layer "F.Cu") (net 6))
 (segment (start 128.04 98) (end 127.9 97.86) (width 0.5) (layer "F.Cu") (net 6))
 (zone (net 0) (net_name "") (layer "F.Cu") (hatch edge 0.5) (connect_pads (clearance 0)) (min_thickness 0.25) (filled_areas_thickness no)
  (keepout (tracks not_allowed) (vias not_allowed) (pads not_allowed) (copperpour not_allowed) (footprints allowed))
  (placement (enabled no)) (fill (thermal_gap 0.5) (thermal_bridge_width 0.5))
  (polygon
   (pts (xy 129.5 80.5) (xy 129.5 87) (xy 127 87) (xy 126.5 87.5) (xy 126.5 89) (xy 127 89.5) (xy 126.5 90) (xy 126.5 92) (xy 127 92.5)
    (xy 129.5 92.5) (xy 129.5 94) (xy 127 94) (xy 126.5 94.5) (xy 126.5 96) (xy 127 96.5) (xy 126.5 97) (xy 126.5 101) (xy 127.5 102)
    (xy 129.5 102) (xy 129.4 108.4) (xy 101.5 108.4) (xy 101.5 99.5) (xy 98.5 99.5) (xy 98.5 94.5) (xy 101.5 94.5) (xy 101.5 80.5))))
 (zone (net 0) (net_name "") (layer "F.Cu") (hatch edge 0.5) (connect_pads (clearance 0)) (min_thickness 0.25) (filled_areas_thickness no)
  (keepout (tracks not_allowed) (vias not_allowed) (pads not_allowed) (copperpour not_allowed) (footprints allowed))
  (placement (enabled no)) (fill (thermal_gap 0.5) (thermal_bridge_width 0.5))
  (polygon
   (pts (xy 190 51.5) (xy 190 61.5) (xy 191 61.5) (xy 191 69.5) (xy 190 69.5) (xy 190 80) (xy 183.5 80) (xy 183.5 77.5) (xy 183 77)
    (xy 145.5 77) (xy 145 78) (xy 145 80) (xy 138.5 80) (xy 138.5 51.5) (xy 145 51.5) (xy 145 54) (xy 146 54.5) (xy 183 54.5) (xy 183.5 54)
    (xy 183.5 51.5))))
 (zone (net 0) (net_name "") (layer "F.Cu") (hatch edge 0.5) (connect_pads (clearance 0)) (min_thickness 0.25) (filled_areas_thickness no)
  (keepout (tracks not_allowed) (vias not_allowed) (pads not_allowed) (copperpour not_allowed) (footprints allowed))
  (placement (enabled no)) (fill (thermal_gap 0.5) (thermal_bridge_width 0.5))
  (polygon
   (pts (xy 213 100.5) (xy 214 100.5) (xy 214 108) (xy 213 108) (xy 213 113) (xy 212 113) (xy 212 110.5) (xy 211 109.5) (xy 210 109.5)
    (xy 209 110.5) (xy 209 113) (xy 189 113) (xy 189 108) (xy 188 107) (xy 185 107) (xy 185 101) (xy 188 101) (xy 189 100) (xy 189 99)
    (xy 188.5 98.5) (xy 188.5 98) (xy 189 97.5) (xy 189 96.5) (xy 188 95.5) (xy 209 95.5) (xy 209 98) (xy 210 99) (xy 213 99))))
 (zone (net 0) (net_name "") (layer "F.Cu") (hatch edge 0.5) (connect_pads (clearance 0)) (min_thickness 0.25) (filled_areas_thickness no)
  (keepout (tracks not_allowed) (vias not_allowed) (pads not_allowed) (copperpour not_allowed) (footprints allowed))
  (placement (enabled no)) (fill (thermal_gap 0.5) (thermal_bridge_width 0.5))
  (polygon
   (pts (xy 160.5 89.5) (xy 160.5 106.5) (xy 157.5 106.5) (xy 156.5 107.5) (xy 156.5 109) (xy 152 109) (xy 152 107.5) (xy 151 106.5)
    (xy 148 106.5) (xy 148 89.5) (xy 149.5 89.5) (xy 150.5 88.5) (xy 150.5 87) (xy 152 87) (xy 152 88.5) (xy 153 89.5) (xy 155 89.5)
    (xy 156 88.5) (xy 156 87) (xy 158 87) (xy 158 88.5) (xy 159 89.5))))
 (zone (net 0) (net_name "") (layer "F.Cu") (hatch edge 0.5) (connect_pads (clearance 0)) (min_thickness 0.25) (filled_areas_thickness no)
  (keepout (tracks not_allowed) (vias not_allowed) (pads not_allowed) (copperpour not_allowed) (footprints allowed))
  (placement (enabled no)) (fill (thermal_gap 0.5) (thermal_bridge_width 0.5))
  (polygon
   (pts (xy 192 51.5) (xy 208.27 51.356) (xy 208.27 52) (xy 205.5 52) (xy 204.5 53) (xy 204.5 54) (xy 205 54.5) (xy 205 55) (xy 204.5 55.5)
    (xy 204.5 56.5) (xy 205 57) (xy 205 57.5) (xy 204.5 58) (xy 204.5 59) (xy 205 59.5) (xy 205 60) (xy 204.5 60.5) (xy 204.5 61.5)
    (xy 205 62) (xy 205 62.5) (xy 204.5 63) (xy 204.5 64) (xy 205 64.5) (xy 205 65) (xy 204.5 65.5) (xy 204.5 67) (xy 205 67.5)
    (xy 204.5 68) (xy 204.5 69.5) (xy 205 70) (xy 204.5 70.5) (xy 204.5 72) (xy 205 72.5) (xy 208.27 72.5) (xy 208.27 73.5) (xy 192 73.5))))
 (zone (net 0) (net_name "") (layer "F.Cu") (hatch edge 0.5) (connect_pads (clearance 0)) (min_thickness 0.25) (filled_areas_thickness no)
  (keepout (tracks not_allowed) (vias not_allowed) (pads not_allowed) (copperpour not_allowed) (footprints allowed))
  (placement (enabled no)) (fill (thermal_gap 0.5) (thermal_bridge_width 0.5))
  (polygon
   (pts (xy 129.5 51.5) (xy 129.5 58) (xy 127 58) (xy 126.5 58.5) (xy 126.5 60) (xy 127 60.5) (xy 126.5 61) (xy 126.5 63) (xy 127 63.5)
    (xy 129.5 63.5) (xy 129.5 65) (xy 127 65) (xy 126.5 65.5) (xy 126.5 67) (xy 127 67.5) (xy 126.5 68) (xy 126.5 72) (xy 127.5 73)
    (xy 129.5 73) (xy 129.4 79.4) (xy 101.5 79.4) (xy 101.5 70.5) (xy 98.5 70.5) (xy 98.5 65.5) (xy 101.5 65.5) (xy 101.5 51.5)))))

